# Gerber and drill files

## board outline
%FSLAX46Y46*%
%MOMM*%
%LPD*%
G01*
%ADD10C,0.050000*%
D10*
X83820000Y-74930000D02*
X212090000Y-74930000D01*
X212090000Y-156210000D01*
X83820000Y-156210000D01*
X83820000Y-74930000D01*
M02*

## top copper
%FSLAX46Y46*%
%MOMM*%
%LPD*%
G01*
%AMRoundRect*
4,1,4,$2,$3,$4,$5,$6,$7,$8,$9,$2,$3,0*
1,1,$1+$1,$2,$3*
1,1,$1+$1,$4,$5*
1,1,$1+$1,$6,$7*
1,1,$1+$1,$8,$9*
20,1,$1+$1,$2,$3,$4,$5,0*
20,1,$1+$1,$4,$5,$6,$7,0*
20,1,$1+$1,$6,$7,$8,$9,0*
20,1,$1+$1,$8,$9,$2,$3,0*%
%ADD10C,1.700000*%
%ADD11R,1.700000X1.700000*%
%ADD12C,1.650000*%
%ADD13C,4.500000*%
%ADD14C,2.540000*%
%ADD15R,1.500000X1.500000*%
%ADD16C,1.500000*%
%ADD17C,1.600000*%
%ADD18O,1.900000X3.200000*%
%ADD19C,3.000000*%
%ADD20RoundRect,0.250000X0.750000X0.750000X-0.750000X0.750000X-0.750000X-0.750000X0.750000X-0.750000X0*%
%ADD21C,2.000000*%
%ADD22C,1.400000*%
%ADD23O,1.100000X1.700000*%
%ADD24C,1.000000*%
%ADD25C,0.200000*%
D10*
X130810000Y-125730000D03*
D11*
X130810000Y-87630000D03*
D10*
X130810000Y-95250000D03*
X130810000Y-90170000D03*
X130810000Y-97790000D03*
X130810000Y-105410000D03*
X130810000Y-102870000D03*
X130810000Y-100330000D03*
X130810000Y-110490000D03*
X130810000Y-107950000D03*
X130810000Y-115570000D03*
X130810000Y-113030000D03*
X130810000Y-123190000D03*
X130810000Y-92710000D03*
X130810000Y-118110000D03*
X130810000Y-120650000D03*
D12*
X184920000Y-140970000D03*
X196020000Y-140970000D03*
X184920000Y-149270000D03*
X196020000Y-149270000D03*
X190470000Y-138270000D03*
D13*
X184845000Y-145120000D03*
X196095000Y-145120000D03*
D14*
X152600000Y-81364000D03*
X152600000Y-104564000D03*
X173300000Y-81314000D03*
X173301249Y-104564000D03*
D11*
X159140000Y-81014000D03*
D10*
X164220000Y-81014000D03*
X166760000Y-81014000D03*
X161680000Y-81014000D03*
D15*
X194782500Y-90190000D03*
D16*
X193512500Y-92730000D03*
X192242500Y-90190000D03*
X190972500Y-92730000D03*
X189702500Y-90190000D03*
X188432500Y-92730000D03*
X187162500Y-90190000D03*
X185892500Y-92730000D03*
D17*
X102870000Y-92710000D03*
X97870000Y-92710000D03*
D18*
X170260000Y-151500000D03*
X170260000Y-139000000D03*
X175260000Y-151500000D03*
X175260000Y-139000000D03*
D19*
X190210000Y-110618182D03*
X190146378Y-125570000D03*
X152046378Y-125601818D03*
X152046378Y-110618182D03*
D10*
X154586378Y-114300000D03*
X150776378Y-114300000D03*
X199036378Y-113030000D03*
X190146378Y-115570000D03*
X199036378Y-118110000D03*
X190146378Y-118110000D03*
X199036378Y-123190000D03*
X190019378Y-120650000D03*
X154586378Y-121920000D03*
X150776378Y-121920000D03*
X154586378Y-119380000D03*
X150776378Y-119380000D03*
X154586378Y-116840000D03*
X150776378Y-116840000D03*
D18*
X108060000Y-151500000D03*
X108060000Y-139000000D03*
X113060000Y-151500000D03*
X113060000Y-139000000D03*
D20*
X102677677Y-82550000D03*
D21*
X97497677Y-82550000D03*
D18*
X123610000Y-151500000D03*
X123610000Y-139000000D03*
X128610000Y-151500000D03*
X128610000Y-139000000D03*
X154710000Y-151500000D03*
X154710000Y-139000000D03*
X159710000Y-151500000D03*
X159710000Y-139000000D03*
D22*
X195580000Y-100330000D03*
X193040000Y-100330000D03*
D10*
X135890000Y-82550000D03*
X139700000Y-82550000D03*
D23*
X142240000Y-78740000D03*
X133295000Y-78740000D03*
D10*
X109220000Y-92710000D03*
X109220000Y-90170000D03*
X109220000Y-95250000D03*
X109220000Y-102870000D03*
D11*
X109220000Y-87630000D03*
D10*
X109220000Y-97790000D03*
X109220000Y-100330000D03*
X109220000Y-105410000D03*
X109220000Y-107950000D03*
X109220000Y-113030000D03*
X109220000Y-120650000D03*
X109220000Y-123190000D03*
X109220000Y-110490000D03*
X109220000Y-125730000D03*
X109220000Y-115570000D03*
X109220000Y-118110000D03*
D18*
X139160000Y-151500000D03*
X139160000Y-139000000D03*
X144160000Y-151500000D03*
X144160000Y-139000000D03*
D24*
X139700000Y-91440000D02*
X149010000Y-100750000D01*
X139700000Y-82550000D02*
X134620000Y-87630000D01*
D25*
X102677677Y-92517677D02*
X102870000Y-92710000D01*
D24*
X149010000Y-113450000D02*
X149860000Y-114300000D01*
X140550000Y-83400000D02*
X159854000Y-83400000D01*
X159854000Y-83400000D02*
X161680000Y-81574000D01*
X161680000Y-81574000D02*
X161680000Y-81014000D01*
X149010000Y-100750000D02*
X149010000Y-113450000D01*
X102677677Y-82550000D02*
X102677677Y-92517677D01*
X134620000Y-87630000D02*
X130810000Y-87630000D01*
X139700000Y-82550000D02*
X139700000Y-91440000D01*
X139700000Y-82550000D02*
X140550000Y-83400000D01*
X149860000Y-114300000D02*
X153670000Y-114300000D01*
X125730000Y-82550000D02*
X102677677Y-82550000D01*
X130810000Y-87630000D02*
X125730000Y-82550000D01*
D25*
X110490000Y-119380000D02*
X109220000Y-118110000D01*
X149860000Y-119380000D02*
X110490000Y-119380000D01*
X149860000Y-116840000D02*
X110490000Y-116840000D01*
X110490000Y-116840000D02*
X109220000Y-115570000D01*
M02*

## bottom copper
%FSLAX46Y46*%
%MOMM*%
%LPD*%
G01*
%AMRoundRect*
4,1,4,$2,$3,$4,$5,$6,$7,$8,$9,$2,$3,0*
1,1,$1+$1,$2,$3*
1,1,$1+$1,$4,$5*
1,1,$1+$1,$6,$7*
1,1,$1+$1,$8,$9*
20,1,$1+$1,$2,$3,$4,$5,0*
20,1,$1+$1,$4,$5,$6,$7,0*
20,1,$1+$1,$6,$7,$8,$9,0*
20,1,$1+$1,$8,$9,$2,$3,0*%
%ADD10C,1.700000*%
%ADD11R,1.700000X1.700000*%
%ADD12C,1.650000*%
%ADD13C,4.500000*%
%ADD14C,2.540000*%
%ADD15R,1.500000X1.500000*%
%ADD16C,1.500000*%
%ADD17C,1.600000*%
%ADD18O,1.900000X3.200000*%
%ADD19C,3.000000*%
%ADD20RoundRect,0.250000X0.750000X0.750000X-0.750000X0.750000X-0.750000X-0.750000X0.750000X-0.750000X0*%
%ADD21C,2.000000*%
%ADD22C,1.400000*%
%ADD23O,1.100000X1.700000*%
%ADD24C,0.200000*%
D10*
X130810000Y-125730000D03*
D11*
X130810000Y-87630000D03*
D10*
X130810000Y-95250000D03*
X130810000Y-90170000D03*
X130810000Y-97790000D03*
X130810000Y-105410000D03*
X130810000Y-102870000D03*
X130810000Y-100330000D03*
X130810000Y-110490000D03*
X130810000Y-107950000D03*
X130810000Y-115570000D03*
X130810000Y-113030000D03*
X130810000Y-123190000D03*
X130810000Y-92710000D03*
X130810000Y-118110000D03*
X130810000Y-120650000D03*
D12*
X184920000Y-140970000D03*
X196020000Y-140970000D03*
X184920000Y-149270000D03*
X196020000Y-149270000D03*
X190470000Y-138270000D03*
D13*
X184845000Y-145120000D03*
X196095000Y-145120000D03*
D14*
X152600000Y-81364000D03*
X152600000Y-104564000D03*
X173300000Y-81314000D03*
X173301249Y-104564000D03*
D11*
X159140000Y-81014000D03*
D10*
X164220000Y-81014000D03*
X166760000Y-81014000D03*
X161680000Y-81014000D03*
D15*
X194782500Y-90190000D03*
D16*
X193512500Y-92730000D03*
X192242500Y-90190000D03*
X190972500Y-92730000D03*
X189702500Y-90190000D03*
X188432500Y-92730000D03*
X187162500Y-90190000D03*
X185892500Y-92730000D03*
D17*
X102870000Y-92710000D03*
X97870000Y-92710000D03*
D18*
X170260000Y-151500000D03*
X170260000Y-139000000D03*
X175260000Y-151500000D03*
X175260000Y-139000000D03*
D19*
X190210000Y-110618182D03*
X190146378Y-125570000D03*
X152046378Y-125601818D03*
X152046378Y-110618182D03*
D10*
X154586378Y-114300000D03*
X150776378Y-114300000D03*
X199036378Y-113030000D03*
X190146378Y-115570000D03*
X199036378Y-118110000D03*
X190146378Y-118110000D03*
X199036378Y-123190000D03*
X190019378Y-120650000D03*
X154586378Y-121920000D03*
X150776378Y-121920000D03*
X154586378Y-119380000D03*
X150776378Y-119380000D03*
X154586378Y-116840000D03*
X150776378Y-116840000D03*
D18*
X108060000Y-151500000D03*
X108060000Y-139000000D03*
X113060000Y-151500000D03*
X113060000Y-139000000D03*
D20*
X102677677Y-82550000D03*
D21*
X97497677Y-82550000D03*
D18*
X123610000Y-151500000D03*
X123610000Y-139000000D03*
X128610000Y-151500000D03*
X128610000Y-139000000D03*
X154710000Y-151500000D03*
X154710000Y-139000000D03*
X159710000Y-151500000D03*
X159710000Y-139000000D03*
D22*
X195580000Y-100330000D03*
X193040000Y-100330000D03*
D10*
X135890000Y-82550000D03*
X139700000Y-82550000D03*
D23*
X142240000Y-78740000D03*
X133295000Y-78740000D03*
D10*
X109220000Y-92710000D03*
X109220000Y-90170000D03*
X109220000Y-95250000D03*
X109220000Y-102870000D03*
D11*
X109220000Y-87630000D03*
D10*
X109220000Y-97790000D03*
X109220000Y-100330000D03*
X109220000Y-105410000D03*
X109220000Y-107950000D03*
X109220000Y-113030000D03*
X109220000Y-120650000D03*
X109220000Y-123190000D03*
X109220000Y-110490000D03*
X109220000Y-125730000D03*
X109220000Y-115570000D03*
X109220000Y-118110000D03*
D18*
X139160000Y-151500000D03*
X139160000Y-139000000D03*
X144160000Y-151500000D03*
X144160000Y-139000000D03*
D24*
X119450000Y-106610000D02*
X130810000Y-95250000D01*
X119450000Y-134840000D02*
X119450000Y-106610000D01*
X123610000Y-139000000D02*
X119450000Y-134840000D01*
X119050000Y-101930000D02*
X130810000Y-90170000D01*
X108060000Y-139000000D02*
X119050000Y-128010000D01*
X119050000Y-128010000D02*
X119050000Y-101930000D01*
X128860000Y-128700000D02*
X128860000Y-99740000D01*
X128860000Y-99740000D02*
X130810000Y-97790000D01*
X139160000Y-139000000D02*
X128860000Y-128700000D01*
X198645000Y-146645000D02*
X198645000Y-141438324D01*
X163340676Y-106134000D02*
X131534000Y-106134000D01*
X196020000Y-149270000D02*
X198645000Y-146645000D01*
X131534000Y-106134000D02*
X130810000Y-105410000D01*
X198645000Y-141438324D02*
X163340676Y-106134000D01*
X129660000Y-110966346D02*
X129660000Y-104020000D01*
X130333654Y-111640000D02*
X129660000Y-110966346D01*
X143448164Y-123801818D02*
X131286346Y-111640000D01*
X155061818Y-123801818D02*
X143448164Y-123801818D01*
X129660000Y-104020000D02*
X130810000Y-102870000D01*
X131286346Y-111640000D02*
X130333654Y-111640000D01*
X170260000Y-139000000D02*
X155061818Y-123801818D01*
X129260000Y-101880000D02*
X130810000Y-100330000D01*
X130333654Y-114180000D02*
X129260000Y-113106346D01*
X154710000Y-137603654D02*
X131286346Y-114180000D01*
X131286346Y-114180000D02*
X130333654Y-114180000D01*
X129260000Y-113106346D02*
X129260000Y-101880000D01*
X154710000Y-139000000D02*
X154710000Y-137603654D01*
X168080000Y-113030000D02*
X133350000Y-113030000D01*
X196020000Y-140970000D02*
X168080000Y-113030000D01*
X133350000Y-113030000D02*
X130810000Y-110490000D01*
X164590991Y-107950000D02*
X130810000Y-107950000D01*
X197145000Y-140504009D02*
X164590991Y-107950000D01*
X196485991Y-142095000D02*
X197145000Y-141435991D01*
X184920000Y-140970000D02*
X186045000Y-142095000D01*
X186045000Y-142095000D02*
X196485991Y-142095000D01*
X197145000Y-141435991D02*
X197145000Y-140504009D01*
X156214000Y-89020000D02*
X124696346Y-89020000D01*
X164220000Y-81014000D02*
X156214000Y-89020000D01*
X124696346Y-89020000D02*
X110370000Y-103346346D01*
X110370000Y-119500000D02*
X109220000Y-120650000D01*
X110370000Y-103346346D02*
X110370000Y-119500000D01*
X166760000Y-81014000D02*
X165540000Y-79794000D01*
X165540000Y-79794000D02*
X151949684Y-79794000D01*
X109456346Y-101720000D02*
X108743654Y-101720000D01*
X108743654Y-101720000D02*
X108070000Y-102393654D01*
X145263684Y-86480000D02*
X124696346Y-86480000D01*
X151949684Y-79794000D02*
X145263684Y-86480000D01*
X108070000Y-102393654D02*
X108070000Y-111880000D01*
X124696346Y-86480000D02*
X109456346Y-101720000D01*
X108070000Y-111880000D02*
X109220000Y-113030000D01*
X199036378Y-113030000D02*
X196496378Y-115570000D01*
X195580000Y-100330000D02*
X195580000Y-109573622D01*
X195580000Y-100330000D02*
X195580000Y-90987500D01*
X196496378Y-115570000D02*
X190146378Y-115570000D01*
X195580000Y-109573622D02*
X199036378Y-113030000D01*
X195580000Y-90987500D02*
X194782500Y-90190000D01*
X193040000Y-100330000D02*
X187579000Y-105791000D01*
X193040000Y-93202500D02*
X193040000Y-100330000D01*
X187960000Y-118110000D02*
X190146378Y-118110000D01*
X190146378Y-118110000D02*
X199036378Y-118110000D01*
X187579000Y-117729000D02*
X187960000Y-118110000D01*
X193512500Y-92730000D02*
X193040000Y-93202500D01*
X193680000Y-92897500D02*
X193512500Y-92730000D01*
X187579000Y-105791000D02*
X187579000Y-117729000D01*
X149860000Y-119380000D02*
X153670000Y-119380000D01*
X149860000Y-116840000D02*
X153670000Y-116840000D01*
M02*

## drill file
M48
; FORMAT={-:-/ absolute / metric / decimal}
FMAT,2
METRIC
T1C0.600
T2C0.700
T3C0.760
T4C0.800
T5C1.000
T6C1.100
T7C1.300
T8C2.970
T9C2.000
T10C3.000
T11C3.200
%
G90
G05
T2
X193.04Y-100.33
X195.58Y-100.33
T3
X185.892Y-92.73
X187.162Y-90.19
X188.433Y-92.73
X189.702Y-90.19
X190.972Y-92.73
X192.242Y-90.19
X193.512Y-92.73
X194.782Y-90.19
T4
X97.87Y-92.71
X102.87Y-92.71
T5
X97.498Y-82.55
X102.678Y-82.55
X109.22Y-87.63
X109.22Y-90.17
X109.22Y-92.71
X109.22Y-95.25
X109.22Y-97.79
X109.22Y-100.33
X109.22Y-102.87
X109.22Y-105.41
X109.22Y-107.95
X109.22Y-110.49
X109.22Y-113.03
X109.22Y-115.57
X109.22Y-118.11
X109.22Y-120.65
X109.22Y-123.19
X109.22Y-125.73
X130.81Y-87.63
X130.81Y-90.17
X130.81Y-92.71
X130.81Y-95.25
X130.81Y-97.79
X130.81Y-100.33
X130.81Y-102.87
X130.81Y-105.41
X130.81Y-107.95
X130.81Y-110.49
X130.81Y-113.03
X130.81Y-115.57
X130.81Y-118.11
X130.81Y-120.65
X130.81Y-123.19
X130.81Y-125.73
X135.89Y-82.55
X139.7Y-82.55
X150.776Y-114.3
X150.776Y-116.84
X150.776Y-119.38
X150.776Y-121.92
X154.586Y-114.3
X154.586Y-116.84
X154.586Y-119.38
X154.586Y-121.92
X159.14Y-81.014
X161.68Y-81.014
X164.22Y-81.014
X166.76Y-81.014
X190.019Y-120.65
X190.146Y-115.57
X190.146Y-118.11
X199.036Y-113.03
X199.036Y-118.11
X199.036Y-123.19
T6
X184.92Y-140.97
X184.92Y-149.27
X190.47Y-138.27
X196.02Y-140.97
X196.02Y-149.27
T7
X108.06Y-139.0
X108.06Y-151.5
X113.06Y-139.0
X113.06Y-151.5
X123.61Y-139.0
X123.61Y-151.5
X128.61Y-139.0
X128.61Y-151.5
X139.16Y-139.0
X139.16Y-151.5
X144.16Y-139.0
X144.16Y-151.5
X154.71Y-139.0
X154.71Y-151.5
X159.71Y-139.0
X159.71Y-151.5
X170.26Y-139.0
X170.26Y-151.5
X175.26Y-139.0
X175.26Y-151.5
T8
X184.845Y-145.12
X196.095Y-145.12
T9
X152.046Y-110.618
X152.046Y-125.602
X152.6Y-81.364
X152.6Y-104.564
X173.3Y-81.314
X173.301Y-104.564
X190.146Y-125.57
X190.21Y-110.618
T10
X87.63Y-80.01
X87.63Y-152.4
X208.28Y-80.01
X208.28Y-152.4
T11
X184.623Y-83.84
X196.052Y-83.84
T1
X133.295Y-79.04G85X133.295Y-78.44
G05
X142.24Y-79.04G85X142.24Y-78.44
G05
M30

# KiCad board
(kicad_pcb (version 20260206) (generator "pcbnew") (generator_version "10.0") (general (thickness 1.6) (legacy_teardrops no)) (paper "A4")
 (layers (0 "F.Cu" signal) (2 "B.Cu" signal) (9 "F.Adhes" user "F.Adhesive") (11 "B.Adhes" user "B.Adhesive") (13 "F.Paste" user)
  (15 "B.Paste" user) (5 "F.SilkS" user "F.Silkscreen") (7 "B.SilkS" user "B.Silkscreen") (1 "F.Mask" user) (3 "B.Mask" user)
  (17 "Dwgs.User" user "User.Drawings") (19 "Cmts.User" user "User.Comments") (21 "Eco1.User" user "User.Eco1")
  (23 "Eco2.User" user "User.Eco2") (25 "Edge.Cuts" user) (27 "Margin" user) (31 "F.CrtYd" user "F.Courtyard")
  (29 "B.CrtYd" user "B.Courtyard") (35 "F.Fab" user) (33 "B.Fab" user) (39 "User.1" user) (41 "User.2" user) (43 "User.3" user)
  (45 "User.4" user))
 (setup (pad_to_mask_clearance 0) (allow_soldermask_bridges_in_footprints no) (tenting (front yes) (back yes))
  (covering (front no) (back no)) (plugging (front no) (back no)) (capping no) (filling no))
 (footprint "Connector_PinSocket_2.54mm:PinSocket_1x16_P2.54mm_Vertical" (layer "F.Cu") (at 130.81 87.63)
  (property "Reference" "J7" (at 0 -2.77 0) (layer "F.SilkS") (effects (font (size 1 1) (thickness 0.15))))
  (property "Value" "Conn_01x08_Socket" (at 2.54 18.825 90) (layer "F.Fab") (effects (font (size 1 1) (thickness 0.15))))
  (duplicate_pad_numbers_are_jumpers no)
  (pad "3V3" thru_hole circle (at 0 38.1) (size 1.7 1.7) (drill 1) (layers "*.Cu" "*.Mask") (remove_unused_layers no)
   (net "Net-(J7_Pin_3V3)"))
  (pad "5V" thru_hole rect (at 0 0) (size 1.7 1.7) (drill 1) (layers "*.Cu" "*.Mask") (remove_unused_layers no) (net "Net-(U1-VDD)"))
  (pad "12" thru_hole circle (at 0 7.62) (size 1.7 1.7) (drill 1) (layers "*.Cu" "*.Mask") (remove_unused_layers no)
   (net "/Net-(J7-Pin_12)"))
  (pad "13" thru_hole circle (at 0 2.54) (size 1.7 1.7) (drill 1) (layers "*.Cu" "*.Mask") (remove_unused_layers no)
   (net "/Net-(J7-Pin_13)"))
  (pad "14" thru_hole circle (at 0 10.16) (size 1.7 1.7) (drill 1) (layers "*.Cu" "*.Mask") (remove_unused_layers no)
   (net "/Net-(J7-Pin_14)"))
  (pad "25" thru_hole circle (at 0 17.78) (size 1.7 1.7) (drill 1) (layers "*.Cu" "*.Mask") (remove_unused_layers no)
   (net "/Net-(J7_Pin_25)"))
  (pad "26" thru_hole circle (at 0 15.24) (size 1.7 1.7) (drill 1) (layers "*.Cu" "*.Mask") (remove_unused_layers no)
   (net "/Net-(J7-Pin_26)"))
  (pad "27" thru_hole circle (at 0 12.7) (size 1.7 1.7) (drill 1) (layers "*.Cu" "*.Mask") (remove_unused_layers no)
   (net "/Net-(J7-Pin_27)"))
  (pad "32" thru_hole circle (at 0 22.86) (size 1.7 1.7) (drill 1) (layers "*.Cu" "*.Mask") (remove_unused_layers no)
   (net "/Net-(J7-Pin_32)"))
  (pad "33" thru_hole circle (at 0 20.32) (size 1.7 1.7) (drill 1) (layers "*.Cu" "*.Mask") (remove_unused_layers no)
   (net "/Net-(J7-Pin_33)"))
  (pad "34" thru_hole circle (at 0 27.94) (size 1.7 1.7) (drill 1) (layers "*.Cu" "*.Mask") (remove_unused_layers no))
  (pad "35" thru_hole circle (at 0 25.4) (size 1.7 1.7) (drill 1) (layers "*.Cu" "*.Mask") (remove_unused_layers no))
  (pad "EN" thru_hole circle (at 0 35.56) (size 1.7 1.7) (drill 1) (layers "*.Cu" "*.Mask") (remove_unused_layers no))
  (pad "GND" thru_hole circle (at 0 5.08) (size 1.7 1.7) (drill 1) (layers "*.Cu" "*.Mask") (remove_unused_layers no) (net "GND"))
  (pad "SVN" thru_hole circle (at 0 30.48) (size 1.7 1.7) (drill 1) (layers "*.Cu" "*.Mask") (remove_unused_layers no))
  (pad "SVP" thru_hole circle (at 0 33.02) (size 1.7 1.7) (drill 1) (layers "*.Cu" "*.Mask") (remove_unused_layers no)))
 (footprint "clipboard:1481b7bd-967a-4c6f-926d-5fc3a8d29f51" (layer "F.Cu") (at 199.345 152.37)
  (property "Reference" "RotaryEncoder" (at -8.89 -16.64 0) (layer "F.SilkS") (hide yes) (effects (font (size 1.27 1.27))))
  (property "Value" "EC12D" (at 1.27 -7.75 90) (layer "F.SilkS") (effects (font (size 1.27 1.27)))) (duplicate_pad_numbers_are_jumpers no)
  (pad "A1" thru_hole circle (at -14.425 -11.4) (size 1.65 1.65) (drill 1.1) (layers "*.Cu" "*.Mask") (remove_unused_layers no)
   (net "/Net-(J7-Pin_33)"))
  (pad "B1" thru_hole circle (at -3.325 -11.4) (size 1.65 1.65) (drill 1.1) (layers "*.Cu" "*.Mask") (remove_unused_layers no)
   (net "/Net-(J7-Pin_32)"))
  (pad "C1" thru_hole circle (at -14.425 -3.1) (size 1.65 1.65) (drill 1.1) (layers "*.Cu" "*.Mask") (remove_unused_layers no) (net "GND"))
  (pad "D1" thru_hole circle (at -3.325 -3.1) (size 1.65 1.65) (drill 1.1) (layers "*.Cu" "*.Mask") (remove_unused_layers no)
   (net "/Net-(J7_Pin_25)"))
  (pad "E1" thru_hole circle (at -8.875 -14.1) (size 1.65 1.65) (drill 1.1) (layers "*.Cu" "*.Mask") (remove_unused_layers no) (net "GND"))
  (pad "MH1" thru_hole circle (at -14.5 -7.25) (size 4.5 4.5) (drill 2.97) (layers "*.Cu" "*.Mask") (remove_unused_layers no) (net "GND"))
  (pad "MH2" thru_hole circle (at -3.25 -7.25) (size 4.5 4.5) (drill 2.97) (layers "*.Cu" "*.Mask") (remove_unused_layers no) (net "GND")))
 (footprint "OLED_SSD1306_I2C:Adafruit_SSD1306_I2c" (layer "F.Cu") (at 152.6 81.364)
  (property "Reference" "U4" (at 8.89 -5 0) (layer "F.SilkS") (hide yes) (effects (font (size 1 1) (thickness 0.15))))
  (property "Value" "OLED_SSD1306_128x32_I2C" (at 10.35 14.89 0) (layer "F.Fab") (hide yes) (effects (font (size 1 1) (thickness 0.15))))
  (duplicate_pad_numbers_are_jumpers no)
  (pad "" np_thru_hole circle (at 0 0) (size 2.54 2.54) (drill 2) (layers "*.Cu" "*.Mask"))
  (pad "" np_thru_hole circle (at 0 23.2) (size 2.54 2.54) (drill 2) (layers "*.Cu" "*.Mask"))
  (pad "" np_thru_hole circle (at 20.7 -0.05) (size 2.54 2.54) (drill 2) (layers "*.Cu" "*.Mask"))
  (pad "" np_thru_hole circle (at 20.701249 23.2) (size 2.54 2.54) (drill 2) (layers "*.Cu" "*.Mask"))
  (pad "GND" thru_hole rect (at 6.54 -0.35) (size 1.7 1.7) (drill 1) (layers "*.Cu" "*.Mask") (remove_unused_layers no) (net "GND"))
  (pad "SCL" thru_hole circle (at 11.62 -0.35) (size 1.7 1.7) (drill 1) (layers "*.Cu" "*.Mask") (remove_unused_layers no)
   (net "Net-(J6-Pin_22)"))
  (pad "SDA" thru_hole circle (at 14.16 -0.35) (size 1.7 1.7) (drill 1) (layers "*.Cu" "*.Mask") (remove_unused_layers no)
   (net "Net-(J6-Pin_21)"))
  (pad "VCC" thru_hole circle (at 9.08 -0.35) (size 1.7 1.7) (drill 1) (layers "*.Cu" "*.Mask") (remove_unused_layers no)
   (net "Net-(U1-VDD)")))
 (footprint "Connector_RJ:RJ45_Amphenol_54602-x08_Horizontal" (layer "F.Cu") (at 194.7825 90.19 180)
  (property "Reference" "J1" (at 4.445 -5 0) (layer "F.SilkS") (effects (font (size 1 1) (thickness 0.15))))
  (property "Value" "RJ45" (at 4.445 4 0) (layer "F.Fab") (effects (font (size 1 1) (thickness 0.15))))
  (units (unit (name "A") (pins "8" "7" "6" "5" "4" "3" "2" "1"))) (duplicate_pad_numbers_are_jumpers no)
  (pad "" np_thru_hole circle (at -1.27 6.35 180) (size 3.2 3.2) (drill 3.2) (layers "*.Cu" "*.Mask"))
  (pad "" np_thru_hole circle (at 10.16 6.35 180) (size 3.2 3.2) (drill 3.2) (layers "*.Cu" "*.Mask"))
  (pad "1" thru_hole rect (at 0 0 180) (size 1.5 1.5) (drill 0.76) (layers "*.Cu" "*.Mask") (remove_unused_layers no) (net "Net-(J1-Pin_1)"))
  (pad "2" thru_hole circle (at 1.27 -2.54 180) (size 1.5 1.5) (drill 0.76) (layers "*.Cu" "*.Mask") (remove_unused_layers no)
   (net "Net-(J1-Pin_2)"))
  (pad "3" thru_hole circle (at 2.54 0 180) (size 1.5 1.5) (drill 0.76) (layers "*.Cu" "*.Mask") (remove_unused_layers no)
   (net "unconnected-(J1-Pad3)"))
  (pad "4" thru_hole circle (at 3.81 -2.54 180) (size 1.5 1.5) (drill 0.76) (layers "*.Cu" "*.Mask") (remove_unused_layers no)
   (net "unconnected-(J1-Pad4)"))
  (pad "5" thru_hole circle (at 5.08 0 180) (size 1.5 1.5) (drill 0.76) (layers "*.Cu" "*.Mask") (remove_unused_layers no)
   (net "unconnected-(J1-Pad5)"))
  (pad "6" thru_hole circle (at 6.35 -2.54 180) (size 1.5 1.5) (drill 0.76) (layers "*.Cu" "*.Mask") (remove_unused_layers no)
   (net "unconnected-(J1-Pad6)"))
  (pad "7" thru_hole circle (at 7.62 0 180) (size 1.5 1.5) (drill 0.76) (layers "*.Cu" "*.Mask") (remove_unused_layers no) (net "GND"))
  (pad "8" thru_hole circle (at 8.89 -2.54 180) (size 1.5 1.5) (drill 0.76) (layers "*.Cu" "*.Mask") (remove_unused_layers no) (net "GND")))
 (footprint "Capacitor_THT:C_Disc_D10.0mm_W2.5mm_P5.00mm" (layer "F.Cu") (at 102.87 92.71 180)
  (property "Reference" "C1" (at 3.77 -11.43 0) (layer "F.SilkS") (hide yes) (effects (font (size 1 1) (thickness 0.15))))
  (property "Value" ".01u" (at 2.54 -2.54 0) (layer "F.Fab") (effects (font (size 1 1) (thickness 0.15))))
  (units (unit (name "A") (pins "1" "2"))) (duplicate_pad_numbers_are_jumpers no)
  (pad "1" thru_hole circle (at 0 0 180) (size 1.6 1.6) (drill 0.8) (layers "*.Cu" "*.Mask") (remove_unused_layers no) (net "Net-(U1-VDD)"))
  (pad "2" thru_hole circle (at 5 0 180) (size 1.6 1.6) (drill 0.8) (layers "*.Cu" "*.Mask") (remove_unused_layers no) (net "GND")))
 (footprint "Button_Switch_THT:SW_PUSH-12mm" (layer "F.Cu") (at 170.26 151.5 90)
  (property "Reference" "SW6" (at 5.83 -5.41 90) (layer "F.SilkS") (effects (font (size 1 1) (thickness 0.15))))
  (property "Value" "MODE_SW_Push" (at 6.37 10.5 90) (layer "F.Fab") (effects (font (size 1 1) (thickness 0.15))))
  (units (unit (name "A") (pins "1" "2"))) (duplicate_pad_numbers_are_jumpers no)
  (pad "1" thru_hole oval (at 0 0 90) (size 3.2 1.9) (drill 1.3) (layers "*.Cu" "*.Mask") (remove_unused_layers no) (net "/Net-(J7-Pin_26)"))
  (pad "1" thru_hole oval (at 12.5 0 90) (size 3.2 1.9) (drill 1.3) (layers "*.Cu" "*.Mask") (remove_unused_layers no)
   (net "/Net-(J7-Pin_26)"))
  (pad "2" thru_hole oval (at 0 5 90) (size 3.2 1.9) (drill 1.3) (layers "*.Cu" "*.Mask") (remove_unused_layers no) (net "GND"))
  (pad "2" thru_hole oval (at 12.5 5 90) (size 3.2 1.9) (drill 1.3) (layers "*.Cu" "*.Mask") (remove_unused_layers no) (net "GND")))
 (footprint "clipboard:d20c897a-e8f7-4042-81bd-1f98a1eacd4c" (layer "F.Cu") (at 147.03 108.11 180)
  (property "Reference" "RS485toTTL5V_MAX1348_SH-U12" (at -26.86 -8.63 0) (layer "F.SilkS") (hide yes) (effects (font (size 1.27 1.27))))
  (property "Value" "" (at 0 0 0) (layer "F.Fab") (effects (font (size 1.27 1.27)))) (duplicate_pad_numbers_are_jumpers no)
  (pad "" np_thru_hole circle (at -43.18 -2.508182 180) (size 3 3) (drill 2) (layers "*.Cu" "*.Mask"))
  (pad "" np_thru_hole circle (at -43.116378 -17.46 180) (size 3 3) (drill 2) (layers "*.Cu" "*.Mask"))
  (pad "" np_thru_hole circle (at -5.016378 -17.491818 180) (size 3 3) (drill 2) (layers "*.Cu" "*.Mask"))
  (pad "" np_thru_hole circle (at -5.016378 -2.508182 180) (size 3 3) (drill 2) (layers "*.Cu" "*.Mask"))
  (pad "5VO" thru_hole circle (at -7.556378 -6.19 180) (size 1.7 1.7) (drill 1) (layers "*.Cu" "*.Mask") (remove_unused_layers no)
   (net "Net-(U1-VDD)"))
  (pad "5VO" thru_hole circle (at -3.746378 -6.19 180) (size 1.7 1.7) (drill 1) (layers "*.Cu" "*.Mask") (remove_unused_layers no)
   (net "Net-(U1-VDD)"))
  (pad "A+" thru_hole circle (at -52.006378 -4.92 180) (size 1.7 1.7) (drill 1) (layers "*.Cu" "*.Mask") (remove_unused_layers no)
   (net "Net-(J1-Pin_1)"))
  (pad "A+" thru_hole circle (at -43.116378 -7.46 180) (size 1.7 1.7) (drill 1) (layers "*.Cu" "*.Mask") (remove_unused_layers no)
   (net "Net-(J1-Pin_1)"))
  (pad "B-" thru_hole circle (at -52.006378 -10 180) (size 1.7 1.7) (drill 1) (layers "*.Cu" "*.Mask") (remove_unused_layers no)
   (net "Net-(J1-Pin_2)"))
  (pad "B-" thru_hole circle (at -43.116378 -10 180) (size 1.7 1.7) (drill 1) (layers "*.Cu" "*.Mask") (remove_unused_layers no)
   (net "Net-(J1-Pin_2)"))
  (pad "GND" thru_hole circle (at -52.006378 -15.08 180) (size 1.7 1.7) (drill 1) (layers "*.Cu" "*.Mask") (remove_unused_layers no)
   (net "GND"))
  (pad "GND" thru_hole circle (at -42.989378 -12.54 180) (size 1.7 1.7) (drill 1) (layers "*.Cu" "*.Mask") (remove_unused_layers no)
   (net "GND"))
  (pad "GND" thru_hole circle (at -7.556378 -13.81 180) (size 1.7 1.7) (drill 1) (layers "*.Cu" "*.Mask") (remove_unused_layers no)
   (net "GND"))
  (pad "GND" thru_hole circle (at -3.746378 -13.81 180) (size 1.7 1.7) (drill 1) (layers "*.Cu" "*.Mask") (remove_unused_layers no)
   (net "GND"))
  (pad "RXD" thru_hole circle (at -7.556378 -11.27 180) (size 1.7 1.7) (drill 1) (layers "*.Cu" "*.Mask") (remove_unused_layers no)
   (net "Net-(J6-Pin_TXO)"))
  (pad "RXD" thru_hole circle (at -3.746378 -11.27 180) (size 1.7 1.7) (drill 1) (layers "*.Cu" "*.Mask") (remove_unused_layers no)
   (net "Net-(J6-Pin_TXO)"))
  (pad "TXD" thru_hole circle (at -7.556378 -8.73 180) (size 1.7 1.7) (drill 1) (layers "*.Cu" "*.Mask") (remove_unused_layers no)
   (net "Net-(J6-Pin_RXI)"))
  (pad "TXD" thru_hole circle (at -3.746378 -8.73 180) (size 1.7 1.7) (drill 1) (layers "*.Cu" "*.Mask") (remove_unused_layers no)
   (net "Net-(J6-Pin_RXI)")))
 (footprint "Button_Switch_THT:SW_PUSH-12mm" (layer "F.Cu") (at 108.06 151.5 90)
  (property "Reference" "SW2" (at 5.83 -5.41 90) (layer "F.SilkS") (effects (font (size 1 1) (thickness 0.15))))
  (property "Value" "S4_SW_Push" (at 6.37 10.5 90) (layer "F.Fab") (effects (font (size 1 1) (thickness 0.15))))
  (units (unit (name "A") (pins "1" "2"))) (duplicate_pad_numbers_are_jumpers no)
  (pad "1" thru_hole oval (at 0 0 90) (size 3.2 1.9) (drill 1.3) (layers "*.Cu" "*.Mask") (remove_unused_layers no))
  (pad "1" thru_hole oval (at 12.5 0 90) (size 3.2 1.9) (drill 1.3) (layers "*.Cu" "*.Mask") (remove_unused_layers no)
   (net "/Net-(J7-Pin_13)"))
  (pad "2" thru_hole oval (at 0 5 90) (size 3.2 1.9) (drill 1.3) (layers "*.Cu" "*.Mask") (remove_unused_layers no) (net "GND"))
  (pad "2" thru_hole oval (at 12.5 5 90) (size 3.2 1.9) (drill 1.3) (layers "*.Cu" "*.Mask") (remove_unused_layers no) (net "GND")))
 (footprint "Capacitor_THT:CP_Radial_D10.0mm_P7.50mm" (layer "F.Cu") (at 103.947677 82.55 180)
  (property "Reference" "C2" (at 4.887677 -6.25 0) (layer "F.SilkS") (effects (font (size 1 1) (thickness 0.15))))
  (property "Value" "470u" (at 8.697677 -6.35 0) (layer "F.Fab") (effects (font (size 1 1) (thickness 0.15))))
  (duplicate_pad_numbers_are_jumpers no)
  (pad "1" thru_hole roundrect (at 1.27 0 180) (size 2 2) (drill 1) (layers "*.Cu" "*.Mask") (remove_unused_layers no)
   (roundrect_rratio 0.125) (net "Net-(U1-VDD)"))
  (pad "2" thru_hole circle (at 6.45 0 180) (size 2 2) (drill 1) (layers "*.Cu" "*.Mask") (remove_unused_layers no) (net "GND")))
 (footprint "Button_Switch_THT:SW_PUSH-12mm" (layer "F.Cu") (at 123.61 151.5 90)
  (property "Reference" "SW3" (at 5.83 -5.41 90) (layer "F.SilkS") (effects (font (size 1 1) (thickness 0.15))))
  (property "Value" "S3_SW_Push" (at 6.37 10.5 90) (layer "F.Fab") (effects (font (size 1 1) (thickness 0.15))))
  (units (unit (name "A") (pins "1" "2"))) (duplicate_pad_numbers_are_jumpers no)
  (pad "1" thru_hole oval (at 0 0 90) (size 3.2 1.9) (drill 1.3) (layers "*.Cu" "*.Mask") (remove_unused_layers no))
  (pad "1" thru_hole oval (at 12.5 0 90) (size 3.2 1.9) (drill 1.3) (layers "*.Cu" "*.Mask") (remove_unused_layers no)
   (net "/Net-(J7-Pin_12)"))
  (pad "2" thru_hole oval (at 0 5 90) (size 3.2 1.9) (drill 1.3) (layers "*.Cu" "*.Mask") (remove_unused_layers no) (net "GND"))
  (pad "2" thru_hole oval (at 12.5 5 90) (size 3.2 1.9) (drill 1.3) (layers "*.Cu" "*.Mask") (remove_unused_layers no) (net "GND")))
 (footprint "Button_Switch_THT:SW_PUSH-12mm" (layer "F.Cu") (at 154.71 151.5 90)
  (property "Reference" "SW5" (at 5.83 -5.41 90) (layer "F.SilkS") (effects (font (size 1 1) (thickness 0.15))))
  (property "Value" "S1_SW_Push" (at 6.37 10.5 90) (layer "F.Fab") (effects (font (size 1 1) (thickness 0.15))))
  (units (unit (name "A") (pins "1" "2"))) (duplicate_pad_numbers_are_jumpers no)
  (pad "1" thru_hole oval (at 0 0 90) (size 3.2 1.9) (drill 1.3) (layers "*.Cu" "*.Mask") (remove_unused_layers no) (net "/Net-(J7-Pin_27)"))
  (pad "1" thru_hole oval (at 12.5 0 90) (size 3.2 1.9) (drill 1.3) (layers "*.Cu" "*.Mask") (remove_unused_layers no)
   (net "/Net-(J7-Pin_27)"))
  (pad "2" thru_hole oval (at 0 5 90) (size 3.2 1.9) (drill 1.3) (layers "*.Cu" "*.Mask") (remove_unused_layers no) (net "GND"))
  (pad "2" thru_hole oval (at 12.5 5 90) (size 3.2 1.9) (drill 1.3) (layers "*.Cu" "*.Mask") (remove_unused_layers no) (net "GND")))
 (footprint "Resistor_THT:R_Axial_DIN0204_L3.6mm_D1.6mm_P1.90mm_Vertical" (layer "F.Cu") (at 195.58 100.33 180)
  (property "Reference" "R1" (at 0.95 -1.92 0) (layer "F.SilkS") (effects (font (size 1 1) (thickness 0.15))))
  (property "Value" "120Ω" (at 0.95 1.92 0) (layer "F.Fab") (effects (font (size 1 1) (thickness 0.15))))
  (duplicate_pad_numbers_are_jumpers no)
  (pad "1" thru_hole circle (at 0 0 180) (size 1.4 1.4) (drill 0.7) (layers "*.Cu" "*.Mask") (remove_unused_layers no)
   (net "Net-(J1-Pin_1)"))
  (pad "2" thru_hole circle (at 2.54 0 180) (size 1.4 1.4) (drill 0.7) (layers "*.Cu" "*.Mask") (remove_unused_layers no)
   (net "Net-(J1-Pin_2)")))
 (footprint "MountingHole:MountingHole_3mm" (layer "F.Cu") (at 208.28 152.4 90)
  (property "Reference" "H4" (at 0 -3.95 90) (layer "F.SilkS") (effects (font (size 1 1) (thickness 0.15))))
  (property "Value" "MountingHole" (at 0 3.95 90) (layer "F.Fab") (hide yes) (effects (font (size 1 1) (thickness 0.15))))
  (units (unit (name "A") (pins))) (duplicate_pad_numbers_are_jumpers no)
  (pad "" np_thru_hole circle (at 0 0 90) (size 3 3) (drill 3) (layers "*.Cu" "*.Mask")))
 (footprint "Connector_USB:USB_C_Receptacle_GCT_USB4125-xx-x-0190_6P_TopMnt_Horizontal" (layer "F.Cu") (at 137.795 77.724 180)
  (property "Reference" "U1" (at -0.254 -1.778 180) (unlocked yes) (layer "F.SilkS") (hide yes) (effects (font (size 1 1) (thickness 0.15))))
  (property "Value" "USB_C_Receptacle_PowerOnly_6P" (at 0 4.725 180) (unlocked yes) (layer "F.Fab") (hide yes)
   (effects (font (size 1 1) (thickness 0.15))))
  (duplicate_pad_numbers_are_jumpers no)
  (pad "5" thru_hole circle (at 1.905 -4.826) (size 1.7 1.7) (drill 1) (layers "*.Cu" "*.Mask") (remove_unused_layers no) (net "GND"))
  (pad "6" thru_hole circle (at -1.905 -4.826) (size 1.7 1.7) (drill 1) (layers "*.Cu" "*.Mask") (remove_unused_layers no)
   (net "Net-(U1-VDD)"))
  (pad "SH" thru_hole oval (at -4.445 -1.016 180) (size 1.1 1.7) (drill oval 0.6 1.2) (layers "*.Cu" "*.Mask" "F.Paste")
   (remove_unused_layers no))
  (pad "SH" thru_hole oval (at 4.5 -1.016 180) (size 1.1 1.7) (drill oval 0.6 1.2) (layers "*.Cu" "*.Mask" "F.Paste")
   (remove_unused_layers no)))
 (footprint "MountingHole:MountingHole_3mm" (layer "F.Cu") (at 208.28 80.01 90)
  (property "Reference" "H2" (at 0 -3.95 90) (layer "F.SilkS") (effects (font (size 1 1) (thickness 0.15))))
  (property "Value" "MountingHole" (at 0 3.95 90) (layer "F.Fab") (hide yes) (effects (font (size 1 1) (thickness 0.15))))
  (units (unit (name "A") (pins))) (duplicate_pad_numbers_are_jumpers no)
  (pad "" np_thru_hole circle (at 0 0 90) (size 3 3) (drill 3) (layers "*.Cu" "*.Mask")))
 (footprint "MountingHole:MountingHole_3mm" (layer "F.Cu") (at 87.63 152.4 90)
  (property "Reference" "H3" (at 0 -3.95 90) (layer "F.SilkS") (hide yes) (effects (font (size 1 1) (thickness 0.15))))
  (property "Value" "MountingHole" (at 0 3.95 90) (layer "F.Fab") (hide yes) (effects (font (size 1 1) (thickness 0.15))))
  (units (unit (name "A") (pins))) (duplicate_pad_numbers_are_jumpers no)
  (pad "" np_thru_hole circle (at 0 0 90) (size 3 3) (drill 3) (layers "*.Cu" "*.Mask")))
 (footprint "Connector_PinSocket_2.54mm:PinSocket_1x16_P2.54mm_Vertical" (layer "F.Cu") (at 109.22 87.63)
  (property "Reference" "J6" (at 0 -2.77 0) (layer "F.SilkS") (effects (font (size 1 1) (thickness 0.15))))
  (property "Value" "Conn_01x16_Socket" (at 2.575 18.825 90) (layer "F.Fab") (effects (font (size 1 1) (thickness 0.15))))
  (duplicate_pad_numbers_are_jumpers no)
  (pad "0" thru_hole circle (at 0 5.08) (size 1.7 1.7) (drill 1) (layers "*.Cu" "*.Mask") (remove_unused_layers no) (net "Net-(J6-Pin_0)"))
  (pad "2" thru_hole circle (at 0 2.54) (size 1.7 1.7) (drill 1) (layers "*.Cu" "*.Mask") (remove_unused_layers no) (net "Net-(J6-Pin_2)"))
  (pad "4" thru_hole circle (at 0 7.62) (size 1.7 1.7) (drill 1) (layers "*.Cu" "*.Mask") (remove_unused_layers no) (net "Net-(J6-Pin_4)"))
  (pad "5" thru_hole circle (at 0 15.24) (size 1.7 1.7) (drill 1) (layers "*.Cu" "*.Mask") (remove_unused_layers no)
   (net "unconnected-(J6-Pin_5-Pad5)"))
  (pad "15" thru_hole rect (at 0 0) (size 1.7 1.7) (drill 1) (layers "*.Cu" "*.Mask") (remove_unused_layers no) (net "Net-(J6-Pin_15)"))
  (pad "16" thru_hole circle (at 0 10.16) (size 1.7 1.7) (drill 1) (layers "*.Cu" "*.Mask") (remove_unused_layers no)
   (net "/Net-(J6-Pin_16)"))
  (pad "17" thru_hole circle (at 0 12.7) (size 1.7 1.7) (drill 1) (layers "*.Cu" "*.Mask") (remove_unused_layers no) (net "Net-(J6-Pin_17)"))
  (pad "18" thru_hole circle (at 0 17.78) (size 1.7 1.7) (drill 1) (layers "*.Cu" "*.Mask") (remove_unused_layers no)
   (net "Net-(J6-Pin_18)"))
  (pad "19" thru_hole circle (at 0 20.32) (size 1.7 1.7) (drill 1) (layers "*.Cu" "*.Mask") (remove_unused_layers no)
   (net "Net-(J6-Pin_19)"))
  (pad "21" thru_hole circle (at 0 25.4) (size 1.7 1.7) (drill 1) (layers "*.Cu" "*.Mask") (remove_unused_layers no) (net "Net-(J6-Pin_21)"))
  (pad "22" thru_hole circle (at 0 33.02) (size 1.7 1.7) (drill 1) (layers "*.Cu" "*.Mask") (remove_unused_layers no)
   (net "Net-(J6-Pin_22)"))
  (pad "23" thru_hole circle (at 0 35.56) (size 1.7 1.7) (drill 1) (layers "*.Cu" "*.Mask") (remove_unused_layers no)
   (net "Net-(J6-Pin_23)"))
  (pad "GND" thru_hole circle (at 0 22.86) (size 1.7 1.7) (drill 1) (layers "*.Cu" "*.Mask") (remove_unused_layers no) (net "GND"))
  (pad "GND" thru_hole circle (at 0 38.1) (size 1.7 1.7) (drill 1) (layers "*.Cu" "*.Mask") (remove_unused_layers no) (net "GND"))
  (pad "RXI" thru_hole circle (at 0 27.94) (size 1.7 1.7) (drill 1) (layers "*.Cu" "*.Mask") (remove_unused_layers no)
   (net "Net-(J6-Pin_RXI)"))
  (pad "TXO" thru_hole circle (at 0 30.48) (size 1.7 1.7) (drill 1) (layers "*.Cu" "*.Mask") (remove_unused_layers no)
   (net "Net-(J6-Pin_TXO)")))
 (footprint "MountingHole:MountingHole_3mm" (layer "F.Cu") (at 87.63 80.01 90)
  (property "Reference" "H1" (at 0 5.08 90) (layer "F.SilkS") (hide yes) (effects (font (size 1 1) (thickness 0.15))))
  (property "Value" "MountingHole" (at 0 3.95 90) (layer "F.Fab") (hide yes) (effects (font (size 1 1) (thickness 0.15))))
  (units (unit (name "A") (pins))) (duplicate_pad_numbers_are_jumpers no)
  (pad "" np_thru_hole circle (at 0 0 90) (size 3 3) (drill 3) (layers "*.Cu" "*.Mask")))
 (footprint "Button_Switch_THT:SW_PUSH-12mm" (layer "F.Cu") (at 139.16 151.5 90)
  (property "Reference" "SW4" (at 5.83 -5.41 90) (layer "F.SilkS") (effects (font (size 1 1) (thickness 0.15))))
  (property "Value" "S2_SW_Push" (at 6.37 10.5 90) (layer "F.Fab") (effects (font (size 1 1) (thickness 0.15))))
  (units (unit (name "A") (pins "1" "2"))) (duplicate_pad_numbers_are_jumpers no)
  (pad "1" thru_hole oval (at 0 0 90) (size 3.2 1.9) (drill 1.3) (layers "*.Cu" "*.Mask") (remove_unused_layers no) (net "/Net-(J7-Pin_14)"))
  (pad "1" thru_hole oval (at 12.5 0 90) (size 3.2 1.9) (drill 1.3) (layers "*.Cu" "*.Mask") (remove_unused_layers no)
   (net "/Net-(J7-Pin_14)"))
  (pad "2" thru_hole oval (at 0 5 90) (size 3.2 1.9) (drill 1.3) (layers "*.Cu" "*.Mask") (remove_unused_layers no) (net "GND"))
  (pad "2" thru_hole oval (at 12.5 5 90) (size 3.2 1.9) (drill 1.3) (layers "*.Cu" "*.Mask") (remove_unused_layers no) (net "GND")))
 (gr_rect (start 83.82 74.93) (end 212.09 156.21) (stroke (width 0.05) (type default)) (fill no) (layer "Edge.Cuts"))
 (segment (start 139.7 91.44) (end 149.01 100.75) (width 1) (layer "F.Cu") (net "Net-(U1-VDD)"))
 (segment (start 139.7 82.55) (end 134.62 87.63) (width 1) (layer "F.Cu") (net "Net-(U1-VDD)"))
 (segment (start 102.677677 92.517677) (end 102.87 92.71) (width 0.2) (layer "F.Cu") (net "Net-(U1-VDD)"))
 (segment (start 149.01 113.45) (end 149.86 114.3) (width 1) (layer "F.Cu") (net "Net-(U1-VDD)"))
 (segment (start 140.55 83.4) (end 159.854 83.4) (width 1) (layer "F.Cu") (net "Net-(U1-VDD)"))
 (segment (start 159.854 83.4) (end 161.68 81.574) (width 1) (layer "F.Cu") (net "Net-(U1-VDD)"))
 (segment (start 161.68 81.574) (end 161.68 81.014) (width 1) (layer "F.Cu") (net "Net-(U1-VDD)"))
 (segment (start 149.01 100.75) (end 149.01 113.45) (width 1) (layer "F.Cu") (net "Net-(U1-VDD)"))
 (segment (start 102.677677 82.55) (end 102.677677 92.517677) (width 1) (layer "F.Cu") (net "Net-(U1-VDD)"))
 (segment (start 134.62 87.63) (end 130.81 87.63) (width 1) (layer "F.Cu") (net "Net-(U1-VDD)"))
 (segment (start 139.7 82.55) (end 139.7 91.44) (width 1) (layer "F.Cu") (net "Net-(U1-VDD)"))
 (segment (start 139.7 82.55) (end 140.55 83.4) (width 1) (layer "F.Cu") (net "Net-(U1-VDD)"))
 (segment (start 149.86 114.3) (end 153.67 114.3) (width 1) (layer "F.Cu") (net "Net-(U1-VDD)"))
 (segment (start 125.73 82.55) (end 102.677677 82.55) (width 1) (layer "F.Cu") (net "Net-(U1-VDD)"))
 (segment (start 130.81 87.63) (end 125.73 82.55) (width 1) (layer "F.Cu") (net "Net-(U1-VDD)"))
 (segment (start 119.45 106.61) (end 130.81 95.25) (width 0.2) (layer "B.Cu") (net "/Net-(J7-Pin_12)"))
 (segment (start 119.45 134.84) (end 119.45 106.61) (width 0.2) (layer "B.Cu") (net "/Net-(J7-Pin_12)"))
 (segment (start 123.61 139) (end 119.45 134.84) (width 0.2) (layer "B.Cu") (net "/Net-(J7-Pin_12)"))
 (segment (start 119.05 101.93) (end 130.81 90.17) (width 0.2) (layer "B.Cu") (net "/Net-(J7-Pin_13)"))
 (segment (start 108.06 139) (end 119.05 128.01) (width 0.2) (layer "B.Cu") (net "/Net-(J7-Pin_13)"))
 (segment (start 119.05 128.01) (end 119.05 101.93) (width 0.2) (layer "B.Cu") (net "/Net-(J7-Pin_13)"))
 (segment (start 128.86 128.7) (end 128.86 99.74) (width 0.2) (layer "B.Cu") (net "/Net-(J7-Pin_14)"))
 (segment (start 128.86 99.74) (end 130.81 97.79) (width 0.2) (layer "B.Cu") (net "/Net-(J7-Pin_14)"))
 (segment (start 139.16 139) (end 128.86 128.7) (width 0.2) (layer "B.Cu") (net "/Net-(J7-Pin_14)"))
 (segment (start 198.645 146.645) (end 198.645 141.438324) (width 0.2) (layer "B.Cu") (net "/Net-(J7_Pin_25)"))
 (segment (start 163.340676 106.134) (end 131.534 106.134) (width 0.2) (layer "B.Cu") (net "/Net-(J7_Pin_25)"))
 (segment (start 196.02 149.27) (end 198.645 146.645) (width 0.2) (layer "B.Cu") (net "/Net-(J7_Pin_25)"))
 (segment (start 131.534 106.134) (end 130.81 105.41) (width 0.2) (layer "B.Cu") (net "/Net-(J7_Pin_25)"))
 (segment (start 198.645 141.438324) (end 163.340676 106.134) (width 0.2) (layer "B.Cu") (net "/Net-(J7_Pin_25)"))
 (segment (start 129.66 110.966346) (end 129.66 104.02) (width 0.2) (layer "B.Cu") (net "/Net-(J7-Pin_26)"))
 (segment (start 130.333654 111.64) (end 129.66 110.966346) (width 0.2) (layer "B.Cu") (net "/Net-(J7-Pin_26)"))
 (segment (start 143.448164 123.801818) (end 131.286346 111.64) (width 0.2) (layer "B.Cu") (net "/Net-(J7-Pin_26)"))
 (segment (start 155.061818 123.801818) (end 143.448164 123.801818) (width 0.2) (layer "B.Cu") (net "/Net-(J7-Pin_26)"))
 (segment (start 129.66 104.02) (end 130.81 102.87) (width 0.2) (layer "B.Cu") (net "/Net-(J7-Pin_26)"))
 (segment (start 131.286346 111.64) (end 130.333654 111.64) (width 0.2) (layer "B.Cu") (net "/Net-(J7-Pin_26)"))
 (segment (start 170.26 139) (end 155.061818 123.801818) (width 0.2) (layer "B.Cu") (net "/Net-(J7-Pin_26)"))
 (segment (start 129.26 101.88) (end 130.81 100.33) (width 0.2) (layer "B.Cu") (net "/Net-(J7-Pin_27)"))
 (segment (start 130.333654 114.18) (end 129.26 113.106346) (width 0.2) (layer "B.Cu") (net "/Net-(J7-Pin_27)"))
 (segment (start 154.71 137.603654) (end 131.286346 114.18) (width 0.2) (layer "B.Cu") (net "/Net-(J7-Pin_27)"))
 (segment (start 131.286346 114.18) (end 130.333654 114.18) (width 0.2) (layer "B.Cu") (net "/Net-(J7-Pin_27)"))
 (segment (start 129.26 113.106346) (end 129.26 101.88) (width 0.2) (layer "B.Cu") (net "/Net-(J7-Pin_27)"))
 (segment (start 154.71 139) (end 154.71 137.603654) (width 0.2) (layer "B.Cu") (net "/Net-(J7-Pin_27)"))
 (segment (start 168.08 113.03) (end 133.35 113.03) (width 0.2) (layer "B.Cu") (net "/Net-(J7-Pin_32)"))
 (segment (start 196.02 140.97) (end 168.08 113.03) (width 0.2) (layer "B.Cu") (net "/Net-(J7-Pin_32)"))
 (segment (start 133.35 113.03) (end 130.81 110.49) (width 0.2) (layer "B.Cu") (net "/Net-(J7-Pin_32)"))
 (segment (start 164.590991 107.95) (end 130.81 107.95) (width 0.2) (layer "B.Cu") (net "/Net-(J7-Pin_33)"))
 (segment (start 197.145 140.504009) (end 164.590991 107.95) (width 0.2) (layer "B.Cu") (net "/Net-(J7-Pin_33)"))
 (segment (start 196.485991 142.095) (end 197.145 141.435991) (width 0.2) (layer "B.Cu") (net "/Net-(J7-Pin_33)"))
 (segment (start 184.92 140.97) (end 186.045 142.095) (width 0.2) (layer "B.Cu") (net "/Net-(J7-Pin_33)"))
 (segment (start 186.045 142.095) (end 196.485991 142.095) (width 0.2) (layer "B.Cu") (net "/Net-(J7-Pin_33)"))
 (segment (start 197.145 141.435991) (end 197.145 140.504009) (width 0.2) (layer "B.Cu") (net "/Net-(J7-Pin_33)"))
 (segment (start 156.214 89.02) (end 124.696346 89.02) (width 0.2) (layer "B.Cu") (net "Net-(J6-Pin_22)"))
 (segment (start 164.22 81.014) (end 156.214 89.02) (width 0.2) (layer "B.Cu") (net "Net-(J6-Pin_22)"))
 (segment (start 124.696346 89.02) (end 110.37 103.346346) (width 0.2) (layer "B.Cu") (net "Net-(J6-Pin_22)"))
 (segment (start 110.37 119.5) (end 109.22 120.65) (width 0.2) (layer "B.Cu") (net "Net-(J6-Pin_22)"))
 (segment (start 110.37 103.346346) (end 110.37 119.5) (width 0.2) (layer "B.Cu") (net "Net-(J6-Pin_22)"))
 (segment (start 166.76 81.014) (end 165.54 79.794) (width 0.2) (layer "B.Cu") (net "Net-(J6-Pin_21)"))
 (segment (start 165.54 79.794) (end 151.949684 79.794) (width 0.2) (layer "B.Cu") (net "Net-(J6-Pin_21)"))
 (segment (start 109.456346 101.72) (end 108.743654 101.72) (width 0.2) (layer "B.Cu") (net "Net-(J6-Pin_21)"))
 (segment (start 108.743654 101.72) (end 108.07 102.393654) (width 0.2) (layer "B.Cu") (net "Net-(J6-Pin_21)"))
 (segment (start 145.263684 86.48) (end 124.696346 86.48) (width 0.2) (layer "B.Cu") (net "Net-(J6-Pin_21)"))
 (segment (start 151.949684 79.794) (end 145.263684 86.48) (width 0.2) (layer "B.Cu") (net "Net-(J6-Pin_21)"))
 (segment (start 108.07 102.393654) (end 108.07 111.88) (width 0.2) (layer "B.Cu") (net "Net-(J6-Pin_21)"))
 (segment (start 124.696346 86.48) (end 109.456346 101.72) (width 0.2) (layer "B.Cu") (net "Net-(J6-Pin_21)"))
 (segment (start 108.07 111.88) (end 109.22 113.03) (width 0.2) (layer "B.Cu") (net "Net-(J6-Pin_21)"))
 (segment (start 199.036378 113.03) (end 196.496378 115.57) (width 0.2) (layer "B.Cu") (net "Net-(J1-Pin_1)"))
 (segment (start 195.58 100.33) (end 195.58 109.573622) (width 0.2) (layer "B.Cu") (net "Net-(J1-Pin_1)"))
 (segment (start 195.58 100.33) (end 195.58 90.9875) (width 0.2) (layer "B.Cu") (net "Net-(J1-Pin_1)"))
 (segment (start 196.496378 115.57) (end 190.146378 115.57) (width 0.2) (layer "B.Cu") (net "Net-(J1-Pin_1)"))
 (segment (start 195.58 109.573622) (end 199.036378 113.03) (width 0.2) (layer "B.Cu") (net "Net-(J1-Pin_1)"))
 (segment (start 195.58 90.9875) (end 194.7825 90.19) (width 0.2) (layer "B.Cu") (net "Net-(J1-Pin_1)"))
 (segment (start 193.04 100.33) (end 187.579 105.791) (width 0.2) (layer "B.Cu") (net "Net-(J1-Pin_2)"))
 (segment (start 193.04 93.2025) (end 193.04 100.33) (width 0.2) (layer "B.Cu") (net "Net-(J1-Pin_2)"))
 (segment (start 187.96 118.11) (end 190.146378 118.11) (width 0.2) (layer "B.Cu") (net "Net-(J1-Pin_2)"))
 (segment (start 190.146378 118.11) (end 199.036378 118.11) (width 0.2) (layer "B.Cu") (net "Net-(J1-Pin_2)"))
 (segment (start 187.579 117.729) (end 187.96 118.11) (width 0.2) (layer "B.Cu") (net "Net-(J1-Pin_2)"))
 (segment (start 193.5125 92.73) (end 193.04 93.2025) (width 0.2) (layer "B.Cu") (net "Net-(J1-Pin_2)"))
 (segment (start 193.68 92.8975) (end 193.5125 92.73) (width 0.2) (layer "B.Cu") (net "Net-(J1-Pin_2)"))
 (segment (start 187.579 105.791) (end 187.579 117.729) (width 0.2) (layer "B.Cu") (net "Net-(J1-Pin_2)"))
 (segment (start 110.49 119.38) (end 109.22 118.11) (width 0.2) (layer "F.Cu") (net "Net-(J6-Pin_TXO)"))
 (segment (start 149.86 119.38) (end 110.49 119.38) (width 0.2) (layer "F.Cu") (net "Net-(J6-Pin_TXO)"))
 (segment (start 149.86 119.38) (end 153.67 119.38) (width 0.2) (layer "B.Cu") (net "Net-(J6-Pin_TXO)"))
 (segment (start 149.86 116.84) (end 110.49 116.84) (width 0.2) (layer "F.Cu") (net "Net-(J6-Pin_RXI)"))
 (segment (start 110.49 116.84) (end 109.22 115.57) (width 0.2) (layer "F.Cu") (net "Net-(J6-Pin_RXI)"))
 (segment (start 149.86 116.84) (end 153.67 116.84) (width 0.2) (layer "B.Cu") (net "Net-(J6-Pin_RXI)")))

